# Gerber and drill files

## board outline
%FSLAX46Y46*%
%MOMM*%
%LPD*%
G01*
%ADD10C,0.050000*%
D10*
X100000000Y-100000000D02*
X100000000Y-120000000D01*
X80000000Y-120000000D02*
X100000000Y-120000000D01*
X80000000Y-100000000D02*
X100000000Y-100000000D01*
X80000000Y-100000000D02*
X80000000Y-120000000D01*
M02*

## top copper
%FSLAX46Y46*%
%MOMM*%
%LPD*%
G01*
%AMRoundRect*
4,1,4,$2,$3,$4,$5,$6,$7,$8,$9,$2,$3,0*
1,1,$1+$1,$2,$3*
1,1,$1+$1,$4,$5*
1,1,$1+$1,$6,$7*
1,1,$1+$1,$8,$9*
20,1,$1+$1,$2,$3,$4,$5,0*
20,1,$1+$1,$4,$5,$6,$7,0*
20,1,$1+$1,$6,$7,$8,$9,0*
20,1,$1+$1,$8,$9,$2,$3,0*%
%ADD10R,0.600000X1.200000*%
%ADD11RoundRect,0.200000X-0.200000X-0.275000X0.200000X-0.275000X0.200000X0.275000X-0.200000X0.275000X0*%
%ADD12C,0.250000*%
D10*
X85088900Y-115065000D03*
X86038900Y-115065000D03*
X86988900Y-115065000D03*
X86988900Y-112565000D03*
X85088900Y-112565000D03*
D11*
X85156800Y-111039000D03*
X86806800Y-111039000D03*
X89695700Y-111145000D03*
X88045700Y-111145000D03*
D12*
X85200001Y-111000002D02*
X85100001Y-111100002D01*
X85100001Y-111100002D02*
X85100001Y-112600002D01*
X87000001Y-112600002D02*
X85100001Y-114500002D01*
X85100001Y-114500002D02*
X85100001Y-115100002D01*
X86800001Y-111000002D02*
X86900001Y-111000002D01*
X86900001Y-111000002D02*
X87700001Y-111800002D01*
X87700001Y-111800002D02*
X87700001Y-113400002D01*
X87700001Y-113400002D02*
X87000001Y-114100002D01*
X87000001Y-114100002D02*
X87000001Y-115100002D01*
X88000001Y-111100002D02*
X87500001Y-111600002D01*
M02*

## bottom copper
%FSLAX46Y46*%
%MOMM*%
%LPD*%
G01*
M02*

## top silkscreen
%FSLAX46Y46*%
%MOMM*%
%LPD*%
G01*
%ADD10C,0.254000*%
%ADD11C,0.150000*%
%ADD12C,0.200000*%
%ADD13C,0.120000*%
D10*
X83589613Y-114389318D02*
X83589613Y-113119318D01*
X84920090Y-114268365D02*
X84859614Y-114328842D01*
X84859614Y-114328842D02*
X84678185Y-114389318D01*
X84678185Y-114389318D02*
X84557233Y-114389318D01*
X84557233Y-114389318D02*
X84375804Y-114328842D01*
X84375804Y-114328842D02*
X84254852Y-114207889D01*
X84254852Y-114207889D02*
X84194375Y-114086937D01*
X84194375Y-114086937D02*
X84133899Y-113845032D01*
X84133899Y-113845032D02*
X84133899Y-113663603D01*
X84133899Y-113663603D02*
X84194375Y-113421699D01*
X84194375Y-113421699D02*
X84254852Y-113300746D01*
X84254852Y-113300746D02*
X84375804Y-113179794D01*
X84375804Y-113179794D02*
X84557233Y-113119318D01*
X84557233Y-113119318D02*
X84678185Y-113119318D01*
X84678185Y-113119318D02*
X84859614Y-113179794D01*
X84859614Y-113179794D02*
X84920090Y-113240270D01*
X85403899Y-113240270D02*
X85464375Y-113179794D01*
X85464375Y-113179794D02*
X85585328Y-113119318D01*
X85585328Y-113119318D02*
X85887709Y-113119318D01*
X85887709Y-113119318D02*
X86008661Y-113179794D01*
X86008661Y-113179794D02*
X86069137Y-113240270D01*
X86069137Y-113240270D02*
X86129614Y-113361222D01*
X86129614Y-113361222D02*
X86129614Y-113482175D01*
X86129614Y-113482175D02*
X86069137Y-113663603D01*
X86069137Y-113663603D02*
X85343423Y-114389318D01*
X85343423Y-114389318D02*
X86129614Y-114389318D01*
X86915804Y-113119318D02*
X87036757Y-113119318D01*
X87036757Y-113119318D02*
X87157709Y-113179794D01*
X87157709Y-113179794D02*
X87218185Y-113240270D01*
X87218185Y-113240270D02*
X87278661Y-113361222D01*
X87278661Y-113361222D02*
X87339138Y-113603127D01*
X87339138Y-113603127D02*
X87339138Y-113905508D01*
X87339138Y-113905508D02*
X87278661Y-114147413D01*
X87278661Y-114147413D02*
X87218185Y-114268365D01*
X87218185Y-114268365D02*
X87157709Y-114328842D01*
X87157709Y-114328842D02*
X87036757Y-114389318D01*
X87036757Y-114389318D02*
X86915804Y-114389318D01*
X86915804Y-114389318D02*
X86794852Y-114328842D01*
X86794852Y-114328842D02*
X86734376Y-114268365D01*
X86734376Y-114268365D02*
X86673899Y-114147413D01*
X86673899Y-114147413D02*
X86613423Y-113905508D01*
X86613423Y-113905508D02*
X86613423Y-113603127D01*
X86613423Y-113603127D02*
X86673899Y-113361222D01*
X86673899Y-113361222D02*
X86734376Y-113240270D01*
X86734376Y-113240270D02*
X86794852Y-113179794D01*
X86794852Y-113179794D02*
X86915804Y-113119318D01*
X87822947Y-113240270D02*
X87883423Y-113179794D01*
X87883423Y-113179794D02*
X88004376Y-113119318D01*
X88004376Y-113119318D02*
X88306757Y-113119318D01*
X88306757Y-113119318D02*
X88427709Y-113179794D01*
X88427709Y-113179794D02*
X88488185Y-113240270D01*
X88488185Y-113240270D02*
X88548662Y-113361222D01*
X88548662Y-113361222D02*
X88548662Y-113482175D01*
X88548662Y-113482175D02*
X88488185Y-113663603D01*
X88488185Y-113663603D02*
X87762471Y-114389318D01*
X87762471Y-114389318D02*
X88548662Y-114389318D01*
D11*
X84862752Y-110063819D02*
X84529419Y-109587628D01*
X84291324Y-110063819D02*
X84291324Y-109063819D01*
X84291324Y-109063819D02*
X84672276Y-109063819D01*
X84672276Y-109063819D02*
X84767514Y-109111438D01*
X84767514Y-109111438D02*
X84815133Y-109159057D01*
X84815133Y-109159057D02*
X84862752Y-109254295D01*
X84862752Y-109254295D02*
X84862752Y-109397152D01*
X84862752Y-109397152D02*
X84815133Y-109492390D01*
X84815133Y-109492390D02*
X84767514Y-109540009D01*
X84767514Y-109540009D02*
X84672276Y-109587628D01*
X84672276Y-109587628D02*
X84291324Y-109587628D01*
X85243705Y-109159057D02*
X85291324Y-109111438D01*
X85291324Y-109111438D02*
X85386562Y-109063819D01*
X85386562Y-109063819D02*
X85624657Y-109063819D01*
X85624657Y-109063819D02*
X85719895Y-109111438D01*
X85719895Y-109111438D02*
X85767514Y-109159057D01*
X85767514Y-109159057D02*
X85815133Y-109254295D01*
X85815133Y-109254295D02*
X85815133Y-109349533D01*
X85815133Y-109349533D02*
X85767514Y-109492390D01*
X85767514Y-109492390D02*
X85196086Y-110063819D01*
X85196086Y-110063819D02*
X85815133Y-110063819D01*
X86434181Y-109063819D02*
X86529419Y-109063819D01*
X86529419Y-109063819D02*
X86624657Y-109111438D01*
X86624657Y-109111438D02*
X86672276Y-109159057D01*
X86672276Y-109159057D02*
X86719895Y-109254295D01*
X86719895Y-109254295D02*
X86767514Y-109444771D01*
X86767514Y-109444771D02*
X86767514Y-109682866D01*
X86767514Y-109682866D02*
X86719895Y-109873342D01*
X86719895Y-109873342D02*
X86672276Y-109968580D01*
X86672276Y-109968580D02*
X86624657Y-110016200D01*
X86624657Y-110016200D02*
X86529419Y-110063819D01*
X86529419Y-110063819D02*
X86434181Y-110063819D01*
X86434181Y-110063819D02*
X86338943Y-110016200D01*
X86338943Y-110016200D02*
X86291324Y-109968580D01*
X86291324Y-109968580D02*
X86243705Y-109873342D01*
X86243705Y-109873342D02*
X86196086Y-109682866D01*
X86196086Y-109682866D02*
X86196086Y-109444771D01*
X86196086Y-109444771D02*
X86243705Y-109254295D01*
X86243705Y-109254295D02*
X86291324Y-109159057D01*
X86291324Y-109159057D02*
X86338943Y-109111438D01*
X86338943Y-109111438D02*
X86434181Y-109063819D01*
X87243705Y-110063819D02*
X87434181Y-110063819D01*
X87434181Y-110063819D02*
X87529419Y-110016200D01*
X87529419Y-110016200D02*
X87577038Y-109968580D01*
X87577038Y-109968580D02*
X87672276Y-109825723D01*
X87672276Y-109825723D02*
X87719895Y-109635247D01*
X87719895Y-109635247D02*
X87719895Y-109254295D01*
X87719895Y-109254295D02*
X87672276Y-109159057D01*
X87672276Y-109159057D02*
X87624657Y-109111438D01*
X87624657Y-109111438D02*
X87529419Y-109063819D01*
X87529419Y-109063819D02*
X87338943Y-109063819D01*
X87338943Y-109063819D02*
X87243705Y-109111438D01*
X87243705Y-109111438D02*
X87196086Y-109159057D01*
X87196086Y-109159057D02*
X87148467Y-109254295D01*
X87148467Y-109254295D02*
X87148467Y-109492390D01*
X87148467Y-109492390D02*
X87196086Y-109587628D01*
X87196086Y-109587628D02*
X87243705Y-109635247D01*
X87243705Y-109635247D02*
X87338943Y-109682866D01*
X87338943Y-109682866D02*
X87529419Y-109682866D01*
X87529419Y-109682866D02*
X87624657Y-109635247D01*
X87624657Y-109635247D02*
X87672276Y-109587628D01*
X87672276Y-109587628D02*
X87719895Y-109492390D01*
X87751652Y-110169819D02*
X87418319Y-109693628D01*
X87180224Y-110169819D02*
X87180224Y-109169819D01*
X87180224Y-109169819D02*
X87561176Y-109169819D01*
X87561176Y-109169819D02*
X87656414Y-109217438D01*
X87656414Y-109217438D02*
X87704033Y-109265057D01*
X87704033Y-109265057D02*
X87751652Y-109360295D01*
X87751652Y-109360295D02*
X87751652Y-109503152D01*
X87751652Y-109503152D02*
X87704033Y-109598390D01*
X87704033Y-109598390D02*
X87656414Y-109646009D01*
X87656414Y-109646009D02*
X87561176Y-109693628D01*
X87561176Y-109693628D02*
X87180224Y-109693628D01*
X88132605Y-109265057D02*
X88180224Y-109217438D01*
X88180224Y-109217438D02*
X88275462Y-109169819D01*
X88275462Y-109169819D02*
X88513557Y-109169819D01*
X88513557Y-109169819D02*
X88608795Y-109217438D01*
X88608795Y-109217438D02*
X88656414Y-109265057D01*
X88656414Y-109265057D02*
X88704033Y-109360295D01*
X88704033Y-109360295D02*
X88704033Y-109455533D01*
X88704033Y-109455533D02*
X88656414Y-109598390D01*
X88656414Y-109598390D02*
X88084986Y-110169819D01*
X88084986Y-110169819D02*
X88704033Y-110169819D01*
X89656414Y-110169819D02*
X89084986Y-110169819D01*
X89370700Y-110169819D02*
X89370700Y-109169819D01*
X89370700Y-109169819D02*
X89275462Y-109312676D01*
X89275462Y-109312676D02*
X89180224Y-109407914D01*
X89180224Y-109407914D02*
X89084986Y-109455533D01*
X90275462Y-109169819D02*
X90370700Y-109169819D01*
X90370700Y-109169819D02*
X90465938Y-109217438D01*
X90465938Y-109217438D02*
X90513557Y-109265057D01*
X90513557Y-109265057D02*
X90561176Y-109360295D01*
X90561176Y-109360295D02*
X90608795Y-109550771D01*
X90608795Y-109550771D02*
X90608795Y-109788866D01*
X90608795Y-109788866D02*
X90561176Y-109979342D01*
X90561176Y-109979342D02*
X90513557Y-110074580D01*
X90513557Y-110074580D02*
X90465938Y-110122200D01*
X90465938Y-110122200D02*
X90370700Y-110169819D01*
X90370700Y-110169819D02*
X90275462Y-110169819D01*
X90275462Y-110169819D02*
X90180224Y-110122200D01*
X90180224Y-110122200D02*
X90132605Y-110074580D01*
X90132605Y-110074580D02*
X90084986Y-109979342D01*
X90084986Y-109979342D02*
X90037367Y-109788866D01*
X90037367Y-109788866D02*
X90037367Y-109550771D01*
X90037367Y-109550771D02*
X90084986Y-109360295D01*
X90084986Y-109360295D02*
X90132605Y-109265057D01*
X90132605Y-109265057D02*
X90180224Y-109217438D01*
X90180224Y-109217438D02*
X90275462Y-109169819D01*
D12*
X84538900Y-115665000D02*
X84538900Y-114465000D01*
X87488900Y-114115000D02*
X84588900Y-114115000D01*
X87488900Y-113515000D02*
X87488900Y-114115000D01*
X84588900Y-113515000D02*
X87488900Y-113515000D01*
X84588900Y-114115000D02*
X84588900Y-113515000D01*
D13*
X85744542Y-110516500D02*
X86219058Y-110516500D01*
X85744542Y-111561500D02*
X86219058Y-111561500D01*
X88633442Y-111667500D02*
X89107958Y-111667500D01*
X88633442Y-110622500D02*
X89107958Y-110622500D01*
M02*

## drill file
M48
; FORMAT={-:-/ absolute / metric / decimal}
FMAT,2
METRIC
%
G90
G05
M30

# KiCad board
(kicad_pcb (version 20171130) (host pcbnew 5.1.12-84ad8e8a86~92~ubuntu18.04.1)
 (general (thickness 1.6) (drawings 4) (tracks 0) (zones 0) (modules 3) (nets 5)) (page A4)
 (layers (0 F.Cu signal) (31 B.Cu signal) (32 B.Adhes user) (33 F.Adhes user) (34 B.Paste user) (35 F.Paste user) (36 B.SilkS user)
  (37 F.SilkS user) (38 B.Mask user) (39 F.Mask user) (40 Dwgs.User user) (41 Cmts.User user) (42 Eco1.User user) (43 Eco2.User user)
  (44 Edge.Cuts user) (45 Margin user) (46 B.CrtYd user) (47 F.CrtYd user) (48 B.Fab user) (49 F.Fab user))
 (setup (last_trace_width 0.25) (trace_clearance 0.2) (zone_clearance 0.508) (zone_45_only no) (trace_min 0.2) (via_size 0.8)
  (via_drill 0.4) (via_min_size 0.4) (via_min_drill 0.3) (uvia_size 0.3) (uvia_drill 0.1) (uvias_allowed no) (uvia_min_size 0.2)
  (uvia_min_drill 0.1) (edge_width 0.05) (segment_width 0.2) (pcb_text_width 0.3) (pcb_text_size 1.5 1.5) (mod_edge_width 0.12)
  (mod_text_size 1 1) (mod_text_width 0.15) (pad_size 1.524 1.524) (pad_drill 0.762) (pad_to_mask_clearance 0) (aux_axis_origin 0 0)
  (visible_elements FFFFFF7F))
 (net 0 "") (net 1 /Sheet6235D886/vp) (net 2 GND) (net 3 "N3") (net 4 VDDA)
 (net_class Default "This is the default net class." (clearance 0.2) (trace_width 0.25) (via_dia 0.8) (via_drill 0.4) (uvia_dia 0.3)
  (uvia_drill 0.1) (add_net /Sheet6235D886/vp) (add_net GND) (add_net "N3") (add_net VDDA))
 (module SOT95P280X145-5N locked (layer F.Cu) (at 86.038900 113.815000 90.000000)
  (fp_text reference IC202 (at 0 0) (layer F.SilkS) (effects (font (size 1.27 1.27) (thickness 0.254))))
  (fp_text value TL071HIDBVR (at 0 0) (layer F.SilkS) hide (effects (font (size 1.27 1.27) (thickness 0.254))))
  (fp_line (start -1.85 -1.5) (end -0.65 -1.5) (layer F.SilkS) (width 0.2))
  (fp_line (start -0.3 1.45) (end -0.3 -1.45) (layer F.SilkS) (width 0.2))
  (fp_line (start 0.3 1.45) (end -0.3 1.45) (layer F.SilkS) (width 0.2))
  (fp_line (start 0.3 -1.45) (end 0.3 1.45) (layer F.SilkS) (width 0.2))
  (fp_line (start -0.3 -1.45) (end 0.3 -1.45) (layer F.SilkS) (width 0.2))
  (pad 1 smd rect (at -1.25 -0.95 180.000000) (size 0.6 1.2) (layers F.Cu F.Mask F.Paste) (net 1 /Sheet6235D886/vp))
  (pad 2 smd rect (at -1.25 0 180.000000) (size 0.6 1.2) (layers F.Cu F.Mask F.Paste) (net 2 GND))
  (pad 3 smd rect (at -1.25 0.95 180.000000) (size 0.6 1.2) (layers F.Cu F.Mask F.Paste) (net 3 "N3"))
  (pad 4 smd rect (at 1.25 0.95 180.000000) (size 0.6 1.2) (layers F.Cu F.Mask F.Paste) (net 1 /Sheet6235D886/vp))
  (pad 5 smd rect (at 1.25 -0.95 180.000000) (size 0.6 1.2) (layers F.Cu F.Mask F.Paste) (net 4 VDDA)))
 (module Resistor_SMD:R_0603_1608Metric (layer F.Cu) (at 85.981800 111.039000)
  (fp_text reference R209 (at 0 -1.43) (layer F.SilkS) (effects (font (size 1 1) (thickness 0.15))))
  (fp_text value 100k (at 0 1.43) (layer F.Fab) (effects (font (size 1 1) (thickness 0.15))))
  (fp_line (start -0.237258 -0.5225) (end 0.237258 -0.5225) (layer F.SilkS) (width 0.12))
  (fp_line (start -0.237258 0.5225) (end 0.237258 0.5225) (layer F.SilkS) (width 0.12))
  (pad 1 smd roundrect (at -0.825 0) (size 0.8 0.95) (layers F.Cu F.Mask F.Paste) (roundrect_rratio 0.25) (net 4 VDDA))
  (pad 2 smd roundrect (at 0.825 0) (size 0.8 0.95) (layers F.Cu F.Mask F.Paste) (roundrect_rratio 0.25) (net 3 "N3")))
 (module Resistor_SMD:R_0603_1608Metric (layer F.Cu) (at 88.870700 111.145000)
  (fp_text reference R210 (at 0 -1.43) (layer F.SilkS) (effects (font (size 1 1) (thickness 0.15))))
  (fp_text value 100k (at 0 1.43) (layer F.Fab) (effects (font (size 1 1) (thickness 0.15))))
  (fp_line (start -0.237258 0.5225) (end 0.237258 0.5225) (layer F.SilkS) (width 0.12))
  (fp_line (start -0.237258 -0.5225) (end 0.237258 -0.5225) (layer F.SilkS) (width 0.12))
  (pad 2 smd roundrect (at 0.825 0) (size 0.8 0.95) (layers F.Cu F.Mask F.Paste) (roundrect_rratio 0.25) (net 2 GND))
  (pad 1 smd roundrect (at -0.825 0) (size 0.8 0.95) (layers F.Cu F.Mask F.Paste) (roundrect_rratio 0.25) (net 3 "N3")))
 (gr_line (start 100 100) (end 100 120) (layer Edge.Cuts) (width 0.05))
 (gr_line (start 80 120) (end 100 120) (layer Edge.Cuts) (width 0.05))
 (gr_line (start 80 100) (end 100 100) (layer Edge.Cuts) (width 0.05))
 (gr_line (start 80 100) (end 80 120) (layer Edge.Cuts) (width 0.05))
 (segment (start 85.200001 111.000002) (end 85.100001 111.100002) (width 0.250000) (layer F.Cu) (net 4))
 (segment (start 85.100001 111.100002) (end 85.100001 112.600002) (width 0.250000) (layer F.Cu) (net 4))
 (segment (start 87.000001 112.600002) (end 85.100001 114.500002) (width 0.250000) (layer F.Cu) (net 1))
 (segment (start 85.100001 114.500002) (end 85.100001 115.100002) (width 0.250000) (layer F.Cu) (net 1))
 (segment (start 86.800001 111.000002) (end 86.900001 111.000002) (width 0.250000) (layer F.Cu) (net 3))
 (segment (start 86.900001 111.000002) (end 87.700001 111.800002) (width 0.250000) (layer F.Cu) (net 3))
 (segment (start 87.700001 111.800002) (end 87.700001 113.400002) (width 0.250000) (layer F.Cu) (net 3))
 (segment (start 87.700001 113.400002) (end 87.000001 114.100002) (width 0.250000) (layer F.Cu) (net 3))
 (segment (start 87.000001 114.100002) (end 87.000001 115.100002) (width 0.250000) (layer F.Cu) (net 3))
 (segment (start 88.000001 111.100002) (end 87.500001 111.600002) (width 0.250000) (layer F.Cu) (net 3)))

